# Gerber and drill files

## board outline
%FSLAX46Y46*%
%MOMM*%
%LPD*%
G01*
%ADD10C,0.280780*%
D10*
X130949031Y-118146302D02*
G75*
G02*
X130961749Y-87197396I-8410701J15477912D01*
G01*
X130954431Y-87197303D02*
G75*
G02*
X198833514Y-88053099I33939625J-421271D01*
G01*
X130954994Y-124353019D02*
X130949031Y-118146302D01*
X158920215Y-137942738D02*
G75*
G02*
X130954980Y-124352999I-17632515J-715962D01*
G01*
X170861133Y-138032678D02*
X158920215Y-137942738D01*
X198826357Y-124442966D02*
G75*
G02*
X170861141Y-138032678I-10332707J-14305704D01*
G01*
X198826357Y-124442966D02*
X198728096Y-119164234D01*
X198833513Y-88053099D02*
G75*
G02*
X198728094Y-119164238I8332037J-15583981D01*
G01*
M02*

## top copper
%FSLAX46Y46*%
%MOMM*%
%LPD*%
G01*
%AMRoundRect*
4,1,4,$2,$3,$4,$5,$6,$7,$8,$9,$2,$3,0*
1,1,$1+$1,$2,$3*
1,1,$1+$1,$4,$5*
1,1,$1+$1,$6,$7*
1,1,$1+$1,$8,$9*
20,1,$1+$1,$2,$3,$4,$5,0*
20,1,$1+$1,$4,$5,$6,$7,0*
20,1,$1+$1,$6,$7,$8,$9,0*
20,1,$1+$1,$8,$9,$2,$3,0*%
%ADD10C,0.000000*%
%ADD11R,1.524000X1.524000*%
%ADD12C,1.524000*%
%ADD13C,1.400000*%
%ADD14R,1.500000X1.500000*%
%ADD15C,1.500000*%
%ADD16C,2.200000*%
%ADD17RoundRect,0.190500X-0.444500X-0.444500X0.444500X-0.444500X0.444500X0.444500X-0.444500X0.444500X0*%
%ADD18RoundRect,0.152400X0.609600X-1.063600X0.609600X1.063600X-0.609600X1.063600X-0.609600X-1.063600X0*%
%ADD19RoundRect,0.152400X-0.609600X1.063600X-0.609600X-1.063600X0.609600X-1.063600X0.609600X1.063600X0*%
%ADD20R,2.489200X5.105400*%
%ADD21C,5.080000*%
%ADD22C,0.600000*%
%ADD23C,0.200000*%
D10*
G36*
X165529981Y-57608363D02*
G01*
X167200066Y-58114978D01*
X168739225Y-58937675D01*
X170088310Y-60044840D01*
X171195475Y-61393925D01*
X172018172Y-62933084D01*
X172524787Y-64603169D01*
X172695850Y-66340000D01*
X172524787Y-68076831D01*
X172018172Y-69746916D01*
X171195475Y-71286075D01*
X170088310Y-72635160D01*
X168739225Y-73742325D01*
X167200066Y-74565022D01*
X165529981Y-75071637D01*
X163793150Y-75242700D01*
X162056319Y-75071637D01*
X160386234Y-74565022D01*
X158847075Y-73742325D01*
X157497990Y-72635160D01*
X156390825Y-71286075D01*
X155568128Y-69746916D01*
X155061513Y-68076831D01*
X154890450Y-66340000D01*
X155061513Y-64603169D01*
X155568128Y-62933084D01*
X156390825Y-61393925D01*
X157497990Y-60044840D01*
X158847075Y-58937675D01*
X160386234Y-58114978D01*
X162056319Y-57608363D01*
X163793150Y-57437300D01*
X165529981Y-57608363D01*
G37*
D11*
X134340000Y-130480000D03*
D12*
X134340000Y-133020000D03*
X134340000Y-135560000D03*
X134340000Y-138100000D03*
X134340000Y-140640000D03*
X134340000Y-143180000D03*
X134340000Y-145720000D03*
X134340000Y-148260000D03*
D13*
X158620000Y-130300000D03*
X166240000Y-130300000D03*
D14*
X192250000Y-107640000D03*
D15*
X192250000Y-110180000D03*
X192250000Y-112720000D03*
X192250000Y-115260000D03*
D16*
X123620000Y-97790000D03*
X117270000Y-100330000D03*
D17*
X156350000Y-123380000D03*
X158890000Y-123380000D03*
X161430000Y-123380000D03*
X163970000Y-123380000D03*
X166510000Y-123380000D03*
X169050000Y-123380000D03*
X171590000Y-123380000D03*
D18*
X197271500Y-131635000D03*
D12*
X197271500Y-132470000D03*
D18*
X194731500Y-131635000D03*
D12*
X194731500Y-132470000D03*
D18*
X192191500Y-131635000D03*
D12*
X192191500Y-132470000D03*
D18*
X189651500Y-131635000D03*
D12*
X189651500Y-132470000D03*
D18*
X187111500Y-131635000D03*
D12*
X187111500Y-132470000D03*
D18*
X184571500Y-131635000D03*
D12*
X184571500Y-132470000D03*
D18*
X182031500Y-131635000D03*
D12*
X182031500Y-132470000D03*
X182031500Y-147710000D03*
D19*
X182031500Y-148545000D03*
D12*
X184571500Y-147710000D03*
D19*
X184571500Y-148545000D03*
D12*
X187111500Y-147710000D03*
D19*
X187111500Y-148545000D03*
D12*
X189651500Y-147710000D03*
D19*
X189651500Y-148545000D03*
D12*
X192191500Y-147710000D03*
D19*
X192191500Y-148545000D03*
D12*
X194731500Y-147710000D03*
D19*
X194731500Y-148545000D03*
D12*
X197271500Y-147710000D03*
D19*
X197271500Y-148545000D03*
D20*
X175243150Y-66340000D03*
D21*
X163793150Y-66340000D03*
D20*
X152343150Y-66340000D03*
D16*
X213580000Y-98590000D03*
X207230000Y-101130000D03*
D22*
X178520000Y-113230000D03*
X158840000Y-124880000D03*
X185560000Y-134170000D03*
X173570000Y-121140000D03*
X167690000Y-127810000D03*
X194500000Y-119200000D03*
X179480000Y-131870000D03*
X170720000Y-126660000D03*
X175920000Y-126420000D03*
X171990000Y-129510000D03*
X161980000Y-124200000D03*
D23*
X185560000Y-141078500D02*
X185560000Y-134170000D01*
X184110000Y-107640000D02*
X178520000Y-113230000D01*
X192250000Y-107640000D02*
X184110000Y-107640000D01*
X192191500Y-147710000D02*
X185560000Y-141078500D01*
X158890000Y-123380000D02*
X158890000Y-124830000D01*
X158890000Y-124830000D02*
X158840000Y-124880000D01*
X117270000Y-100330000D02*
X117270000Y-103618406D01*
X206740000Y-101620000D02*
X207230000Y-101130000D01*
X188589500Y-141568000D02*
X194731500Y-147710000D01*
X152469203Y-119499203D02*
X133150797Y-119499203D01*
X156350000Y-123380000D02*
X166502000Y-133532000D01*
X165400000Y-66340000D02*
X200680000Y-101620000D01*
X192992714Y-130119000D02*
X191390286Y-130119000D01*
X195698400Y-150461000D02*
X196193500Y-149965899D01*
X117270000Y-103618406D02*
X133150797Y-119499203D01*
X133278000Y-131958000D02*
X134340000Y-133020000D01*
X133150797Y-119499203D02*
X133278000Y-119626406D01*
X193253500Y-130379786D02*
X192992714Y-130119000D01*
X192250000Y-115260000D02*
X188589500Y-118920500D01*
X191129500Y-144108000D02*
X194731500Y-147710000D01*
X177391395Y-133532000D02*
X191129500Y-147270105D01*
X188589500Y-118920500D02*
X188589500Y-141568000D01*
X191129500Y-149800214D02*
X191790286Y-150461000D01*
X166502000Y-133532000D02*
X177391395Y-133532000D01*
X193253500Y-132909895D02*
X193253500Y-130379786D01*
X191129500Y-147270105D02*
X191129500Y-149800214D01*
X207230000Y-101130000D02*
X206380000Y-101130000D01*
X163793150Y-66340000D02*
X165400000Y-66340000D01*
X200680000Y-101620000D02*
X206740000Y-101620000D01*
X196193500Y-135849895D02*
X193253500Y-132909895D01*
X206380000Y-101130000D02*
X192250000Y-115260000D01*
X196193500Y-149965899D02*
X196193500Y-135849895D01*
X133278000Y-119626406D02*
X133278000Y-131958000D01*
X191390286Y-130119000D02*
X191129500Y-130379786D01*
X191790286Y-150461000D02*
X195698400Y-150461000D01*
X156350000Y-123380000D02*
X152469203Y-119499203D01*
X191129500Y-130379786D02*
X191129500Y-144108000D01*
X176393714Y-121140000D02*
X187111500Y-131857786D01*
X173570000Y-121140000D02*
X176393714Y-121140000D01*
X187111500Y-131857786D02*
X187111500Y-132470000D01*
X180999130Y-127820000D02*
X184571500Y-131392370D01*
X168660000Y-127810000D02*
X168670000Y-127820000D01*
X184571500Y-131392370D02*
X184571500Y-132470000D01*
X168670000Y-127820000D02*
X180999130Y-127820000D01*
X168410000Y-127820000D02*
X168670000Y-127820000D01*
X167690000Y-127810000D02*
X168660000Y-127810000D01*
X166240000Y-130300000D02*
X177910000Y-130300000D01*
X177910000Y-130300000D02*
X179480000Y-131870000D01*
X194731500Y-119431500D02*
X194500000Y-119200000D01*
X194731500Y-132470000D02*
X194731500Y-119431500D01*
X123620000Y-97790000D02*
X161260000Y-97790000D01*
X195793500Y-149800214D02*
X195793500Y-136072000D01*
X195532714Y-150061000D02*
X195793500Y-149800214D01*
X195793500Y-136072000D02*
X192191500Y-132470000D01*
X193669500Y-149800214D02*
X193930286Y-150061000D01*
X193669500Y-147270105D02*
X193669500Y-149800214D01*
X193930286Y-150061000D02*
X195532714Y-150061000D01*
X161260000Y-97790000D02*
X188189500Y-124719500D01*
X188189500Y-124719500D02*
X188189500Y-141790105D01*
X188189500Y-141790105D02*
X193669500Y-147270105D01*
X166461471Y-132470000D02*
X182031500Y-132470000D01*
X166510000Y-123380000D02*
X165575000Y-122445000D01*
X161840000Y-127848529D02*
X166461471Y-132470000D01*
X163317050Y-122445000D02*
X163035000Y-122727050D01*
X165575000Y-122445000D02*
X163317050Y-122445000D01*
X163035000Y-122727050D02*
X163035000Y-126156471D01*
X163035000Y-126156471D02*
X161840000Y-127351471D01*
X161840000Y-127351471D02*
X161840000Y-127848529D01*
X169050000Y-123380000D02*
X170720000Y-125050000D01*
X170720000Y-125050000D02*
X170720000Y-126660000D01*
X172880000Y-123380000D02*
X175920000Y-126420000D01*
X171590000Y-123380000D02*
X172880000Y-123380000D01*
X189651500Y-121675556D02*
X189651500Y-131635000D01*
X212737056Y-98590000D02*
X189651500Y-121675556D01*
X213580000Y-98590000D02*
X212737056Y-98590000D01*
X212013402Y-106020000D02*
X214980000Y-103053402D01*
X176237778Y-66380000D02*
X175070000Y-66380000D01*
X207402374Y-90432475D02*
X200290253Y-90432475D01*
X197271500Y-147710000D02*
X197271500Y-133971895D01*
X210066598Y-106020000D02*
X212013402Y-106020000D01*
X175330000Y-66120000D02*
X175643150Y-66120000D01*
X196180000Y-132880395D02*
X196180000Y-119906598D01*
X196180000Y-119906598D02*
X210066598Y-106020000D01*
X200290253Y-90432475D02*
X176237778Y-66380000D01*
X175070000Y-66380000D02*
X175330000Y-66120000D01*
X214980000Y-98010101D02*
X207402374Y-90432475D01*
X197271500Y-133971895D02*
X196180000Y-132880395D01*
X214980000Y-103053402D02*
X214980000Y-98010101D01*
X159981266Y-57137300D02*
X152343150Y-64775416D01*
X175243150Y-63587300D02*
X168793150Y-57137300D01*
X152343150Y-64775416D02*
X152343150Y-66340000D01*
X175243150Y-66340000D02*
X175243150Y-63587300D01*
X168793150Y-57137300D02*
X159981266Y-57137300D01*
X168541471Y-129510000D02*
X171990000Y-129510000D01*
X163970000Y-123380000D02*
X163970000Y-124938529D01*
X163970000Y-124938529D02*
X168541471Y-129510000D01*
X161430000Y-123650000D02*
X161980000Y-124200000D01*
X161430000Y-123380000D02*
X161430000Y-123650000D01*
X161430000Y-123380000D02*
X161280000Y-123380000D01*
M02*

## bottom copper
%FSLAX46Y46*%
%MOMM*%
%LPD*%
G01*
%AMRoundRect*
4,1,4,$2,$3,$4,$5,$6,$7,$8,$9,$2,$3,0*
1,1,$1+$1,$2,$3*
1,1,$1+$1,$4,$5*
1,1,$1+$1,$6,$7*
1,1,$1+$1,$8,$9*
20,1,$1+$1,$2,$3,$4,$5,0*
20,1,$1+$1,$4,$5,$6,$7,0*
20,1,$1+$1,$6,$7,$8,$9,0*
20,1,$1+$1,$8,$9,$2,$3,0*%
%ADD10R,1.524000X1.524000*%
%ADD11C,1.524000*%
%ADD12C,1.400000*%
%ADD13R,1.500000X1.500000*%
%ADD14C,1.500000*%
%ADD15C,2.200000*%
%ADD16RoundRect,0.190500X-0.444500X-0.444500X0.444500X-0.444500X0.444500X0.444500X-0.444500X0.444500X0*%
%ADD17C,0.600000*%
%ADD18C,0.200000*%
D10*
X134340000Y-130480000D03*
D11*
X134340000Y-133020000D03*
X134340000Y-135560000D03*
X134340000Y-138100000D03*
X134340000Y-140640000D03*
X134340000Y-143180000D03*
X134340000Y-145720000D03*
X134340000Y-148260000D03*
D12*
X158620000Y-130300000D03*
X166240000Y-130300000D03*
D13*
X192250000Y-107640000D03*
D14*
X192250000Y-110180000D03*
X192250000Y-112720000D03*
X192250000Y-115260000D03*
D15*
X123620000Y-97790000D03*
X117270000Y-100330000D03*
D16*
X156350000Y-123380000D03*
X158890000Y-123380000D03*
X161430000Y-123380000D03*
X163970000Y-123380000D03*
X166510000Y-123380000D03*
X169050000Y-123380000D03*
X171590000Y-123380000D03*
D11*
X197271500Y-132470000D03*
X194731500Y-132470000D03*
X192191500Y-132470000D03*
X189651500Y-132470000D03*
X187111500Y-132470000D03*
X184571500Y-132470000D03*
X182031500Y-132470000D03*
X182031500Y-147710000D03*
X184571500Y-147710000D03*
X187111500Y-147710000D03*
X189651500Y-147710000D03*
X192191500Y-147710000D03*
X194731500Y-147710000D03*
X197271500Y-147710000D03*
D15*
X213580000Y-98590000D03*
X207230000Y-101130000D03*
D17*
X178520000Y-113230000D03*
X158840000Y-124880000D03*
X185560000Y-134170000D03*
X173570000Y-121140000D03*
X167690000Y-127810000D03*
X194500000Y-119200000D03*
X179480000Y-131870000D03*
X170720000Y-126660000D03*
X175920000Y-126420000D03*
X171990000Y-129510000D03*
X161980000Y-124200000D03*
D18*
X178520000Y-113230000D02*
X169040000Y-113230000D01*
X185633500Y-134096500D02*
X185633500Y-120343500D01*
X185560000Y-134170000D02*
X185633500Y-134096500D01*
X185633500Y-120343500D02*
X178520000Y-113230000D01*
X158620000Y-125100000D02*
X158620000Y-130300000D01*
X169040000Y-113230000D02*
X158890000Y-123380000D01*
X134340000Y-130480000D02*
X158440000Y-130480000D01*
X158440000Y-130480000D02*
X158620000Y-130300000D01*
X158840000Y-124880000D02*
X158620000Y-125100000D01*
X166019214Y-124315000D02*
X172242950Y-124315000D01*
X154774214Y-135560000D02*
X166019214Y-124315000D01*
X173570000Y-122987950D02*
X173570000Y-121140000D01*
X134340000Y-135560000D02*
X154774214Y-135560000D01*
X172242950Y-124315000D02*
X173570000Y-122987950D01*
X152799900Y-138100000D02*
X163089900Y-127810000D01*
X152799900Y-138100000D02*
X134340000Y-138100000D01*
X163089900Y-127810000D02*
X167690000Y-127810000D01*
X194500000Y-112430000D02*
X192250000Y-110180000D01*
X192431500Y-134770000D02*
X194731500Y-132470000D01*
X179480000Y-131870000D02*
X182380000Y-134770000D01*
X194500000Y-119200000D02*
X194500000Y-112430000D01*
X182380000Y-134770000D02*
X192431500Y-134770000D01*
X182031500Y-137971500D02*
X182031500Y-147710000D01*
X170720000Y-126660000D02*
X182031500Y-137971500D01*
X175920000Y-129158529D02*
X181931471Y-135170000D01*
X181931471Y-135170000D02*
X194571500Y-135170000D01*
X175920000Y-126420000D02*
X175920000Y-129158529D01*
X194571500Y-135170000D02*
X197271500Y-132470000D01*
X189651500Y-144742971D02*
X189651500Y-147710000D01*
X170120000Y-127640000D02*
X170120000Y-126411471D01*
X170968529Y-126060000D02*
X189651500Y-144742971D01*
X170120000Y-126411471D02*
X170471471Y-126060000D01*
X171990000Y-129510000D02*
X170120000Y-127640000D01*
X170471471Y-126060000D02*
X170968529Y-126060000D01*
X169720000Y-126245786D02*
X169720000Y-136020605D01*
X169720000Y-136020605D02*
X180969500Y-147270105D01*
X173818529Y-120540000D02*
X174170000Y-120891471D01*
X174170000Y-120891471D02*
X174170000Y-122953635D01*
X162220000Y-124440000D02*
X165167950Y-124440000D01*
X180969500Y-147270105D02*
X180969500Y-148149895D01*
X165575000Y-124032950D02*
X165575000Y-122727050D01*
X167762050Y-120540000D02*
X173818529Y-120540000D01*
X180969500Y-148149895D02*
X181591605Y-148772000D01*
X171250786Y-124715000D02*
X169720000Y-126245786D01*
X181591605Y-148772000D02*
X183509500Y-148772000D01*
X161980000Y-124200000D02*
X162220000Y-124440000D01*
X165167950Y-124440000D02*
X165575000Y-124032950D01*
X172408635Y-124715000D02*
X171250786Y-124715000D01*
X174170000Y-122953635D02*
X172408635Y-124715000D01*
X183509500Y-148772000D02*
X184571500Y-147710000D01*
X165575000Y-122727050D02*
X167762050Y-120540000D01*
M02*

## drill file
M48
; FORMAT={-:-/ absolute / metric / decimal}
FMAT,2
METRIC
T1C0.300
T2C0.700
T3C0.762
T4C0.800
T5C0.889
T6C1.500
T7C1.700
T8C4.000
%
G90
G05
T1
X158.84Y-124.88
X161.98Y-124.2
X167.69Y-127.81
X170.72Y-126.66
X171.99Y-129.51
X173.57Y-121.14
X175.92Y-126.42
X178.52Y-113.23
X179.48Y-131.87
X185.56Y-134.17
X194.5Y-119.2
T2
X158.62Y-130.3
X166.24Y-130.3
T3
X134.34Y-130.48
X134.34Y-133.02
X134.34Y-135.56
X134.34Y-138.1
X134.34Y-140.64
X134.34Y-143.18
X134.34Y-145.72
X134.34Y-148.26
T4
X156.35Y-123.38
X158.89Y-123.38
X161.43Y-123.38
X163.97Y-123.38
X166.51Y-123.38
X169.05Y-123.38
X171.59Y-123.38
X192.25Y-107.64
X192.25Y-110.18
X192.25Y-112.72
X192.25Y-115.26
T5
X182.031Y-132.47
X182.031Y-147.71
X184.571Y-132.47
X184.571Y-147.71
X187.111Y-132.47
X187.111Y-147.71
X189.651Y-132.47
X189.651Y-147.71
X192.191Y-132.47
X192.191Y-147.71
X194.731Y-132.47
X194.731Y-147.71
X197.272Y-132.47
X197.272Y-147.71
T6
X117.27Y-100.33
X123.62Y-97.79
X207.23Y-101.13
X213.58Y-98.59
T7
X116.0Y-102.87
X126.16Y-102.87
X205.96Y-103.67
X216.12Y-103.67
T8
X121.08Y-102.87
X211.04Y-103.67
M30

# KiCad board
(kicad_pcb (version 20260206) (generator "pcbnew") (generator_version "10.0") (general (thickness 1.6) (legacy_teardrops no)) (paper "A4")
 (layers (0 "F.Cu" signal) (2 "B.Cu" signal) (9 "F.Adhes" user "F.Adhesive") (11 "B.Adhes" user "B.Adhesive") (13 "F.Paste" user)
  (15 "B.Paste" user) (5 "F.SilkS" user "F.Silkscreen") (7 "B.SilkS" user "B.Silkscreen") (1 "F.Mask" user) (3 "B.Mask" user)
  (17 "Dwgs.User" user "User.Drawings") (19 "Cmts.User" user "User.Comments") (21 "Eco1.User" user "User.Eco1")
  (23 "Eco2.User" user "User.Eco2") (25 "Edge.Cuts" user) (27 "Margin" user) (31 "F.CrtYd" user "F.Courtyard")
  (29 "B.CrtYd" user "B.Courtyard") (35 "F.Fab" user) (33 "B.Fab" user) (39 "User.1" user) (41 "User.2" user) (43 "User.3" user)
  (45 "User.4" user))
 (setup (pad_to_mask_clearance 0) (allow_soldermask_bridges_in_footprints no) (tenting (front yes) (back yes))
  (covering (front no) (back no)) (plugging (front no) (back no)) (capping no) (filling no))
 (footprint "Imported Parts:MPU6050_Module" (layer "F.Cu") (at 134.34 130.48)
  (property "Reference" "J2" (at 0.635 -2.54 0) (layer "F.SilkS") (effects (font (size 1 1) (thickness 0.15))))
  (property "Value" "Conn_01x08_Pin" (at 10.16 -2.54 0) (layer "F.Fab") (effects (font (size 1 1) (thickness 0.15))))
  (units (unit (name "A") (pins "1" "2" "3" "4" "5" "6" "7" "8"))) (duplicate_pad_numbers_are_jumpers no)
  (pad "1" thru_hole rect (at 0 0) (size 1.524 1.524) (drill 0.762) (layers "*.Cu" "*.Mask") (remove_unused_layers no) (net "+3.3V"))
  (pad "2" thru_hole circle (at 0 2.54) (size 1.524 1.524) (drill 0.762) (layers "*.Cu" "*.Mask") (remove_unused_layers no) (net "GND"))
  (pad "3" thru_hole circle (at 0 5.08) (size 1.524 1.524) (drill 0.762) (layers "*.Cu" "*.Mask") (remove_unused_layers no) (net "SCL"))
  (pad "4" thru_hole circle (at 0 7.62) (size 1.524 1.524) (drill 0.762) (layers "*.Cu" "*.Mask") (remove_unused_layers no) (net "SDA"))
  (pad "5" thru_hole circle (at 0 10.16) (size 1.524 1.524) (drill 0.762) (layers "*.Cu" "*.Mask") (remove_unused_layers no)
   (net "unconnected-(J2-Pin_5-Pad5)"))
  (pad "6" thru_hole circle (at 0 12.7) (size 1.524 1.524) (drill 0.762) (layers "*.Cu" "*.Mask") (remove_unused_layers no)
   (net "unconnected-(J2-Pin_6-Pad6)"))
  (pad "7" thru_hole circle (at 0 15.24) (size 1.524 1.524) (drill 0.762) (layers "*.Cu" "*.Mask") (remove_unused_layers no)
   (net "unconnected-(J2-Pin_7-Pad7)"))
  (pad "8" thru_hole circle (at 0 17.78) (size 1.524 1.524) (drill 0.762) (layers "*.Cu" "*.Mask") (remove_unused_layers no)
   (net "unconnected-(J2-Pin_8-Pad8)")))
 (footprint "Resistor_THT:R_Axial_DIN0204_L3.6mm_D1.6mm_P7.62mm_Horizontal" (layer "F.Cu") (at 158.62 130.3)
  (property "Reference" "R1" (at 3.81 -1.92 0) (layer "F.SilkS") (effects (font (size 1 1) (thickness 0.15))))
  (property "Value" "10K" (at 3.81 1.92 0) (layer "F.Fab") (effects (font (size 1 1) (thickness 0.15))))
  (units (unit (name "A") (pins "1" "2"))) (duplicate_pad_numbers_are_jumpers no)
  (pad "1" thru_hole circle (at 0 0) (size 1.4 1.4) (drill 0.7) (layers "*.Cu" "*.Mask") (remove_unused_layers no) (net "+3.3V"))
  (pad "2" thru_hole circle (at 7.62 0) (size 1.4 1.4) (drill 0.7) (layers "*.Cu" "*.Mask") (remove_unused_layers no) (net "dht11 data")))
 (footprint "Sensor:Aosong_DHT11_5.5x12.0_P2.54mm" (layer "F.Cu") (at 192.25 107.64)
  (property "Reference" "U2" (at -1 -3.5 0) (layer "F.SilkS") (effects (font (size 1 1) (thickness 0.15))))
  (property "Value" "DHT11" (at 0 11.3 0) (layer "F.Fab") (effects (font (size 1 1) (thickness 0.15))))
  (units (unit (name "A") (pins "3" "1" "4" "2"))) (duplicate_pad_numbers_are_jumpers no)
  (pad "1" thru_hole rect (at 0 0) (size 1.5 1.5) (drill 0.8) (layers "*.Cu" "*.Mask") (remove_unused_layers no) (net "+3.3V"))
  (pad "2" thru_hole circle (at 0 2.54) (size 1.5 1.5) (drill 0.8) (layers "*.Cu" "*.Mask") (remove_unused_layers no) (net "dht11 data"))
  (pad "3" thru_hole circle (at 0 5.08) (size 1.5 1.5) (drill 0.8) (layers "*.Cu" "*.Mask") (remove_unused_layers no)
   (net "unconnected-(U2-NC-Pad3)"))
  (pad "4" thru_hole circle (at 0 7.62) (size 1.5 1.5) (drill 0.8) (layers "*.Cu" "*.Mask") (remove_unused_layers no) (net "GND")))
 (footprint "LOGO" (layer "F.Cu") (at 148.84 83.94)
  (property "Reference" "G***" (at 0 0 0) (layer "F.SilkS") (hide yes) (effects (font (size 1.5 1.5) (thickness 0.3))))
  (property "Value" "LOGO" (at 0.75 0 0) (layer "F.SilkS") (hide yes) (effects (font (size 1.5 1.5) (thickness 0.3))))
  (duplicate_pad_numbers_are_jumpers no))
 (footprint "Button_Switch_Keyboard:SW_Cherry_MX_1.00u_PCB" (layer "F.Cu") (at 123.62 97.79)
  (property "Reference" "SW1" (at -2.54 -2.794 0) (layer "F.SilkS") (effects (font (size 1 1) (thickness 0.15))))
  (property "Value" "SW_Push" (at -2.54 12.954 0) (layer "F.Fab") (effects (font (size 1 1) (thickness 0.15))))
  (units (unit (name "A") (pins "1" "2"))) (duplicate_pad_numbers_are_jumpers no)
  (pad "" np_thru_hole circle (at -7.62 5.08) (size 1.7 1.7) (drill 1.7) (layers "*.Cu" "*.Mask"))
  (pad "" np_thru_hole circle (at -2.54 5.08) (size 4 4) (drill 4) (layers "*.Cu" "*.Mask"))
  (pad "" np_thru_hole circle (at 2.54 5.08) (size 1.7 1.7) (drill 1.7) (layers "*.Cu" "*.Mask"))
  (pad "1" thru_hole circle (at 0 0) (size 2.2 2.2) (drill 1.5) (layers "*.Cu" "*.Mask") (remove_unused_layers no) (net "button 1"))
  (pad "2" thru_hole circle (at -6.35 2.54) (size 2.2 2.2) (drill 1.5) (layers "*.Cu" "*.Mask") (remove_unused_layers no) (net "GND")))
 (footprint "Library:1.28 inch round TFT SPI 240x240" (layer "F.Cu") (at 163.97 98.94)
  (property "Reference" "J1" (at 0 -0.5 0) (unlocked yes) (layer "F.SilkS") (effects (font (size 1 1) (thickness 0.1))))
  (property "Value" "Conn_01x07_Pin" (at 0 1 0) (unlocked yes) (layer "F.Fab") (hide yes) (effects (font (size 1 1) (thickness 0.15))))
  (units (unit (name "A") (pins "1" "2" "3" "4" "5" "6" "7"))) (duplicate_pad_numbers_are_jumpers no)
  (pad "1" thru_hole roundrect (at -7.62 24.44) (size 1.27 1.27) (drill 0.8) (layers "*.Cu" "*.Mask") (remove_unused_layers no)
   (roundrect_rratio 0.15) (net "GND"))
  (pad "2" thru_hole roundrect (at -5.08 24.44) (size 1.27 1.27) (drill 0.8) (layers "*.Cu" "*.Mask") (remove_unused_layers no)
   (roundrect_rratio 0.15) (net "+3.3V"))
  (pad "3" thru_hole roundrect (at -2.54 24.44) (size 1.27 1.27) (drill 0.8) (layers "*.Cu" "*.Mask") (remove_unused_layers no)
   (roundrect_rratio 0.15) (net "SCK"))
  (pad "4" thru_hole roundrect (at 0 24.44) (size 1.27 1.27) (drill 0.8) (layers "*.Cu" "*.Mask") (remove_unused_layers no)
   (roundrect_rratio 0.15) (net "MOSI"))
  (pad "5" thru_hole roundrect (at 2.54 24.44) (size 1.27 1.27) (drill 0.8) (layers "*.Cu" "*.Mask") (remove_unused_layers no)
   (roundrect_rratio 0.15) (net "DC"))
  (pad "6" thru_hole roundrect (at 5.08 24.44) (size 1.27 1.27) (drill 0.8) (layers "*.Cu" "*.Mask") (remove_unused_layers no)
   (roundrect_rratio 0.15) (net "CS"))
  (pad "7" thru_hole roundrect (at 7.62 24.44) (size 1.27 1.27) (drill 0.8) (layers "*.Cu" "*.Mask") (remove_unused_layers no)
   (roundrect_rratio 0.15) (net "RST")))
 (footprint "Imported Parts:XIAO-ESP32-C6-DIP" (layer "F.Cu") (at 189.6515 140.09)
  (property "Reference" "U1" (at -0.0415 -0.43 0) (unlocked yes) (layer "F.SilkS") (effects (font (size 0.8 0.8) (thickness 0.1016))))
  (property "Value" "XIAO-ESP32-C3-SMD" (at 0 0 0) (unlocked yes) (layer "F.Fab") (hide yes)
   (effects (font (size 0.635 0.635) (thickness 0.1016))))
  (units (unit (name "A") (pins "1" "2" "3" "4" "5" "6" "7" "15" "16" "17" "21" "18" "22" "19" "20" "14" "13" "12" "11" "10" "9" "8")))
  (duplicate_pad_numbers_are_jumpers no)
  (pad "1" smd roundrect (at 7.62 -8.455 90) (size 2.432 1.524) (layers "F.Cu" "F.Mask") (roundrect_rratio 0.1) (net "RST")
   (thermal_bridge_angle 45))
  (pad "1" thru_hole circle (at 7.62 -7.62 90) (size 1.524 1.524) (drill 0.889) (layers "*.Cu" "*.Mask") (remove_unused_layers no)
   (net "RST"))
  (pad "2" smd roundrect (at 5.08 -8.455 90) (size 2.432 1.524) (layers "F.Cu" "F.Mask") (roundrect_rratio 0.1) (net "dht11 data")
   (thermal_bridge_angle 45))
  (pad "2" thru_hole circle (at 5.08 -7.62 90) (size 1.524 1.524) (drill 0.889) (layers "*.Cu" "*.Mask") (remove_unused_layers no)
   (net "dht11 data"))
  (pad "3" smd roundrect (at 2.54 -8.455 90) (size 2.432 1.524) (layers "F.Cu" "F.Mask") (roundrect_rratio 0.1) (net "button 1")
   (thermal_bridge_angle 45))
  (pad "3" thru_hole circle (at 2.54 -7.62 90) (size 1.524 1.524) (drill 0.889) (layers "*.Cu" "*.Mask") (remove_unused_layers no)
   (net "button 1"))
  (pad "4" smd roundrect (at 0 -8.455 90) (size 2.432 1.524) (layers "F.Cu" "F.Mask") (roundrect_rratio 0.1) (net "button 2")
   (thermal_bridge_angle 45))
  (pad "4" thru_hole circle (at 0 -7.62 90) (size 1.524 1.524) (drill 0.889) (layers "*.Cu" "*.Mask") (remove_unused_layers no)
   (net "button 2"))
  (pad "5" smd roundrect (at -2.54 -8.455 90) (size 2.432 1.524) (layers "F.Cu" "F.Mask") (roundrect_rratio 0.1) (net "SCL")
   (thermal_bridge_angle 45))
  (pad "5" thru_hole circle (at -2.54 -7.62 90) (size 1.524 1.524) (drill 0.889) (layers "*.Cu" "*.Mask") (remove_unused_layers no)
   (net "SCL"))
  (pad "6" smd roundrect (at -5.08 -8.455 90) (size 2.432 1.524) (layers "F.Cu" "F.Mask") (roundrect_rratio 0.1) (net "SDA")
   (thermal_bridge_angle 45))
  (pad "6" thru_hole circle (at -5.08 -7.62 90) (size 1.524 1.524) (drill 0.889) (layers "*.Cu" "*.Mask") (remove_unused_layers no)
   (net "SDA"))
  (pad "7" smd roundrect (at -7.62 -8.455 90) (size 2.432 1.524) (layers "F.Cu" "F.Mask") (roundrect_rratio 0.1) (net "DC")
   (thermal_bridge_angle 45))
  (pad "7" thru_hole circle (at -7.62 -7.62 90) (size 1.524 1.524) (drill 0.889) (layers "*.Cu" "*.Mask") (remove_unused_layers no)
   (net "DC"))
  (pad "8" thru_hole circle (at -7.62 7.62 270) (size 1.524 1.524) (drill 0.889) (layers "*.Cu" "*.Mask") (remove_unused_layers no)
   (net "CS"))
  (pad "8" smd roundrect (at -7.62 8.455 270) (size 2.432 1.524) (layers "F.Cu" "F.Mask") (roundrect_rratio 0.1) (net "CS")
   (thermal_bridge_angle 45))
  (pad "9" thru_hole circle (at -5.08 7.62 270) (size 1.524 1.524) (drill 0.889) (layers "*.Cu" "*.Mask") (remove_unused_layers no)
   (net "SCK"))
  (pad "9" smd roundrect (at -5.08 8.455 270) (size 2.432 1.524) (layers "F.Cu" "F.Mask") (roundrect_rratio 0.1) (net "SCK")
   (thermal_bridge_angle 45))
  (pad "10" thru_hole circle (at -2.54 7.62 270) (size 1.524 1.524) (drill 0.889) (layers "*.Cu" "*.Mask") (remove_unused_layers no)
   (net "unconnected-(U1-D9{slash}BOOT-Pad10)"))
  (pad "10" smd roundrect (at -2.54 8.455 270) (size 2.432 1.524) (layers "F.Cu" "F.Mask") (roundrect_rratio 0.1)
   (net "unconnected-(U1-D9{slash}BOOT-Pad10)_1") (thermal_bridge_angle 45))
  (pad "11" thru_hole circle (at 0 7.62 270) (size 1.524 1.524) (drill 0.889) (layers "*.Cu" "*.Mask") (remove_unused_layers no)
   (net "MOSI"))
  (pad "11" smd roundrect (at 0 8.455 270) (size 2.432 1.524) (layers "F.Cu" "F.Mask") (roundrect_rratio 0.1) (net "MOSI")
   (thermal_bridge_angle 45))
  (pad "12" thru_hole circle (at 2.54 7.62 270) (size 1.524 1.524) (drill 0.889) (layers "*.Cu" "*.Mask") (remove_unused_layers no)
   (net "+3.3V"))
  (pad "12" smd roundrect (at 2.54 8.455 270) (size 2.432 1.524) (layers "F.Cu" "F.Mask") (roundrect_rratio 0.1) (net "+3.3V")
   (thermal_bridge_angle 45))
  (pad "13" thru_hole circle (at 5.08 7.62 270) (size 1.524 1.524) (drill 0.889) (layers "*.Cu" "*.Mask") (remove_unused_layers no)
   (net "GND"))
  (pad "13" smd roundrect (at 5.08 8.455 270) (size 2.432 1.524) (layers "F.Cu" "F.Mask") (roundrect_rratio 0.1) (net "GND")
   (thermal_bridge_angle 45))
  (pad "14" thru_hole circle (at 7.62 7.62 270) (size 1.524 1.524) (drill 0.889) (layers "*.Cu" "*.Mask") (remove_unused_layers no)
   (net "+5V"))
  (pad "14" smd roundrect (at 7.62 8.455 270) (size 2.432 1.524) (layers "F.Cu" "F.Mask") (roundrect_rratio 0.1) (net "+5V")
   (thermal_bridge_angle 45)))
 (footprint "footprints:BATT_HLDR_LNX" (layer "F.Cu") (at 163.79315 66.34 180)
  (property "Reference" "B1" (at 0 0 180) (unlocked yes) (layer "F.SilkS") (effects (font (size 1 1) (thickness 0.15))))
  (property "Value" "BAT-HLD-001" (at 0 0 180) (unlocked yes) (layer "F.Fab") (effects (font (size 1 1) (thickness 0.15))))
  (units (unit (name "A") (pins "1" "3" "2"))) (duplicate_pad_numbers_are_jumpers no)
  (fp_poly
   (pts (xy 8.9027 0) (xy 8.731637 -1.736831) (xy 8.225022 -3.406916) (xy 7.402325 -4.946075) (xy 6.29516 -6.29516) (xy 4.946075 -7.402325)
    (xy 3.406916 -8.225022) (xy 1.736831 -8.731637) (xy 0 -8.9027) (xy -1.736831 -8.731637) (xy -3.406916 -8.225022)
    (xy -4.946075 -7.402325) (xy -6.29516 -6.29516) (xy -7.402325 -4.946075) (xy -8.225022 -3.406916) (xy -8.731637 -1.736831)
    (xy -8.9027 0) (xy -8.731637 1.736831) (xy -8.225022 3.406916) (xy -7.402325 4.946075) (xy -6.29516 6.29516) (xy -4.946075 7.402325)
    (xy -3.406916 8.225022) (xy -1.736831 8.731637) (xy 0 8.9027) (xy 1.736831 8.731637) (xy 3.406916 8.225022) (xy 4.946075 7.402325)
    (xy 6.29516 6.29516) (xy 7.402325 4.946075) (xy 8.225022 3.406916) (xy 8.731637 1.736831))
   (stroke (width 0) (type solid)) (fill yes) (layer "F.Cu"))
  (pad "1" smd rect (at -11.45 0 180) (size 2.4892 5.1054) (layers "F.Cu" "F.Mask" "F.Paste") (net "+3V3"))
  (pad "2" smd circle (at 0 0 180) (size 5.08 5.08) (layers "F.Cu" "F.Mask" "F.Paste") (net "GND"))
  (pad "3" smd rect (at 11.45 0 180) (size 2.4892 5.1054) (layers "F.Cu" "F.Mask" "F.Paste") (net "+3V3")))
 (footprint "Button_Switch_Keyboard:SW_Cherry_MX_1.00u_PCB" (layer "F.Cu") (at 213.58 98.59)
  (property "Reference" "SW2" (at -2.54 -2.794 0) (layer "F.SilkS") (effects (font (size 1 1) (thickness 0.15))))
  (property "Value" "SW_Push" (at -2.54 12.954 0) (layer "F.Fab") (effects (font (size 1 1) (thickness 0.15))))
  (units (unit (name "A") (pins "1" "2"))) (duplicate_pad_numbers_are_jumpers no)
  (pad "" np_thru_hole circle (at -7.62 5.08) (size 1.7 1.7) (drill 1.7) (layers "*.Cu" "*.Mask"))
  (pad "" np_thru_hole circle (at -2.54 5.08) (size 4 4) (drill 4) (layers "*.Cu" "*.Mask"))
  (pad "" np_thru_hole circle (at 2.54 5.08) (size 1.7 1.7) (drill 1.7) (layers "*.Cu" "*.Mask"))
  (pad "1" thru_hole circle (at 0 0) (size 2.2 2.2) (drill 1.5) (layers "*.Cu" "*.Mask") (remove_unused_layers no) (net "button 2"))
  (pad "2" thru_hole circle (at -6.35 2.54) (size 2.2 2.2) (drill 1.5) (layers "*.Cu" "*.Mask") (remove_unused_layers no) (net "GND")))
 (gr_arc (start 130.949031 118.146302) (mid 104.922837 102.661154) (end 130.961752 87.197391) (stroke (width 0.28078) (type solid))
  (layer "Edge.Cuts"))
 (gr_arc (start 130.954431 87.197303) (mid 165.321951 53.679032) (end 198.833513 88.053099) (stroke (width 0.28078) (type solid))
  (layer "Edge.Cuts"))
 (gr_line (start 130.954994 124.353019) (end 130.949031 118.146302) (stroke (width 0.28078) (type solid)) (layer "Edge.Cuts"))
 (gr_arc (start 158.920215 137.942738) (mid 133.574606 154.530907) (end 130.954994 124.353019) (stroke (width 0.28078) (type solid))
  (layer "Edge.Cuts"))
 (gr_line (start 170.861133 138.032678) (end 158.920215 137.942738) (stroke (width 0.28078) (type solid)) (layer "Edge.Cuts"))
 (gr_arc (start 198.826357 124.442966) (mid 196.20674 154.620857) (end 170.861133 138.032678) (stroke (width 0.28078) (type solid))
  (layer "Edge.Cuts"))
 (gr_line (start 198.826357 124.442966) (end 198.728096 119.164234) (stroke (width 0.28078) (type solid)) (layer "Edge.Cuts"))
 (gr_arc (start 198.833513 88.053099) (mid 224.83698 103.696965) (end 198.728096 119.164234) (stroke (width 0.28078) (type solid))
  (layer "Edge.Cuts"))
 (segment (start 185.56 141.0785) (end 185.56 134.17) (width 0.2) (layer "F.Cu") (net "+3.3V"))
 (segment (start 184.11 107.64) (end 178.52 113.23) (width 0.2) (layer "F.Cu") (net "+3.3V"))
 (segment (start 192.25 107.64) (end 184.11 107.64) (width 0.2) (layer "F.Cu") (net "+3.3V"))
 (segment (start 192.1915 147.71) (end 185.56 141.0785) (width 0.2) (layer "F.Cu") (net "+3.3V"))
 (segment (start 158.89 123.38) (end 158.89 124.83) (width 0.2) (layer "F.Cu") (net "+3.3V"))
 (segment (start 158.89 124.83) (end 158.84 124.88) (width 0.2) (layer "F.Cu") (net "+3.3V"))
 (via (at 178.52 113.23) (size 0.6) (drill 0.3) (layers "F.Cu" "B.Cu") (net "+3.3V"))
 (via (at 158.84 124.88) (size 0.6) (drill 0.3) (layers "F.Cu" "B.Cu") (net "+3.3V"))
 (via (at 185.56 134.17) (size 0.6) (drill 0.3) (layers "F.Cu" "B.Cu") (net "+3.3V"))
 (segment (start 178.52 113.23) (end 169.04 113.23) (width 0.2) (layer "B.Cu") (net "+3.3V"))
 (segment (start 185.6335 134.0965) (end 185.6335 120.3435) (width 0.2) (layer "B.Cu") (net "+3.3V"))
 (segment (start 185.56 134.17) (end 185.6335 134.0965) (width 0.2) (layer "B.Cu") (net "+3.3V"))
 (segment (start 185.6335 120.3435) (end 178.52 113.23) (width 0.2) (layer "B.Cu") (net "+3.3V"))
 (segment (start 158.62 125.1) (end 158.62 130.3) (width 0.2) (layer "B.Cu") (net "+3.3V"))
 (segment (start 169.04 113.23) (end 158.89 123.38) (width 0.2) (layer "B.Cu") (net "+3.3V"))
 (segment (start 134.34 130.48) (end 158.44 130.48) (width 0.2) (layer "B.Cu") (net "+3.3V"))
 (segment (start 158.44 130.48) (end 158.62 130.3) (width 0.2) (layer "B.Cu") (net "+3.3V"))
 (segment (start 158.84 124.88) (end 158.62 125.1) (width 0.2) (layer "B.Cu") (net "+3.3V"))
 (segment (start 117.27 100.33) (end 117.27 103.618406) (width 0.2) (layer "F.Cu") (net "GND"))
 (segment (start 206.74 101.62) (end 207.23 101.13) (width 0.2) (layer "F.Cu") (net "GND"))
 (segment (start 188.5895 141.568) (end 194.7315 147.71) (width 0.2) (layer "F.Cu") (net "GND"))
 (segment (start 152.469203 119.499203) (end 133.150797 119.499203) (width 0.2) (layer "F.Cu") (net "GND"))
 (segment (start 156.35 123.38) (end 166.502 133.532) (width 0.2) (layer "F.Cu") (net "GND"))
 (segment (start 165.4 66.34) (end 200.68 101.62) (width 0.2) (layer "F.Cu") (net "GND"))
 (segment (start 192.992714 130.119) (end 191.390286 130.119) (width 0.2) (layer "F.Cu") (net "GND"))
 (segment (start 195.6984 150.461) (end 196.1935 149.965899) (width 0.2) (layer "F.Cu") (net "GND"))
 (segment (start 117.27 103.618406) (end 133.150797 119.499203) (width 0.2) (layer "F.Cu") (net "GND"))
 (segment (start 133.278 131.958) (end 134.34 133.02) (width 0.2) (layer "F.Cu") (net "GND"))
 (segment (start 133.150797 119.499203) (end 133.278 119.626406) (width 0.2) (layer "F.Cu") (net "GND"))
 (segment (start 193.2535 130.379786) (end 192.992714 130.119) (width 0.2) (layer "F.Cu") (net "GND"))
 (segment (start 192.25 115.26) (end 188.5895 118.9205) (width 0.2) (layer "F.Cu") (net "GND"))
 (segment (start 191.1295 144.108) (end 194.7315 147.71) (width 0.2) (layer "F.Cu") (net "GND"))
 (segment (start 177.391395 133.532) (end 191.1295 147.270105) (width 0.2) (layer "F.Cu") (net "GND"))
 (segment (start 188.5895 118.9205) (end 188.5895 141.568) (width 0.2) (layer "F.Cu") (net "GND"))
 (segment (start 191.1295 149.800214) (end 191.790286 150.461) (width 0.2) (layer "F.Cu") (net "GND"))
 (segment (start 166.502 133.532) (end 177.391395 133.532) (width 0.2) (layer "F.Cu") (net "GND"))
 (segment (start 193.2535 132.909895) (end 193.2535 130.379786) (width 0.2) (layer "F.Cu") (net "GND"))
 (segment (start 191.1295 147.270105) (end 191.1295 149.800214) (width 0.2) (layer "F.Cu") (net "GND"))
 (segment (start 207.23 101.13) (end 206.38 101.13) (width 0.2) (layer "F.Cu") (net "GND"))
 (segment (start 163.79315 66.34) (end 165.4 66.34) (width 0.2) (layer "F.Cu") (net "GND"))
 (segment (start 200.68 101.62) (end 206.74 101.62) (width 0.2) (layer "F.Cu") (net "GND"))
 (segment (start 196.1935 135.849895) (end 193.2535 132.909895) (width 0.2) (layer "F.Cu") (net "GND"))
 (segment (start 206.38 101.13) (end 192.25 115.26) (width 0.2) (layer "F.Cu") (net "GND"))
 (segment (start 196.1935 149.965899) (end 196.1935 135.849895) (width 0.2) (layer "F.Cu") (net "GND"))
 (segment (start 133.278 119.626406) (end 133.278 131.958) (width 0.2) (layer "F.Cu") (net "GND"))
 (segment (start 191.390286 130.119) (end 191.1295 130.379786) (width 0.2) (layer "F.Cu") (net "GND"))
 (segment (start 191.790286 150.461) (end 195.6984 150.461) (width 0.2) (layer "F.Cu") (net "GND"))
 (segment (start 156.35 123.38) (end 152.469203 119.499203) (width 0.2) (layer "F.Cu") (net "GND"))
 (segment (start 191.1295 130.379786) (end 191.1295 144.108) (width 0.2) (layer "F.Cu") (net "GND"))
 (segment (start 176.393714 121.14) (end 187.1115 131.857786) (width 0.2) (layer "F.Cu") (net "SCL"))
 (segment (start 173.57 121.14) (end 176.393714 121.14) (width 0.2) (layer "F.Cu") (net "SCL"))
 (segment (start 187.1115 131.857786) (end 187.1115 132.47) (width 0.2) (layer "F.Cu") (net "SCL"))
 (via (at 173.57 121.14) (size 0.6) (drill 0.3) (layers "F.Cu" "B.Cu") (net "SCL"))
 (segment (start 166.019214 124.315) (end 172.24295 124.315) (width 0.2) (layer "B.Cu") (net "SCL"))
 (segment (start 154.774214 135.56) (end 166.019214 124.315) (width 0.2) (layer "B.Cu") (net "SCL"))
 (segment (start 173.57 122.98795) (end 173.57 121.14) (width 0.2) (layer "B.Cu") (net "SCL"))
 (segment (start 134.34 135.56) (end 154.774214 135.56) (width 0.2) (layer "B.Cu") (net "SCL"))
 (segment (start 172.24295 124.315) (end 173.57 122.98795) (width 0.2) (layer "B.Cu") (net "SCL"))
 (segment (start 180.99913 127.82) (end 184.5715 131.39237) (width 0.2) (layer "F.Cu") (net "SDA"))
 (segment (start 168.66 127.81) (end 168.67 127.82) (width 0.2) (layer "F.Cu") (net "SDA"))
 (segment (start 184.5715 131.39237) (end 184.5715 132.47) (width 0.2) (layer "F.Cu") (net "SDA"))
 (segment (start 168.67 127.82) (end 180.99913 127.82) (width 0.2) (layer "F.Cu") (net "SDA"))
 (segment (start 168.41 127.82) (end 168.67 127.82) (width 0.2) (layer "F.Cu") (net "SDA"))
 (segment (start 167.69 127.81) (end 168.66 127.81) (width 0.2) (layer "F.Cu") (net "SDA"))
 (via (at 167.69 127.81) (size 0.6) (drill 0.3) (layers "F.Cu" "B.Cu") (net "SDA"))
 (segment (start 152.7999 138.1) (end 163.0899 127.81) (width 0.2) (layer "B.Cu") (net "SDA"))
 (segment (start 152.7999 138.1) (end 134.34 138.1) (width 0.2) (layer "B.Cu") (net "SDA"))
 (segment (start 163.0899 127.81) (end 167.69 127.81) (width 0.2) (layer "B.Cu") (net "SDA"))
 (segment (start 166.24 130.3) (end 177.91 130.3) (width 0.2) (layer "F.Cu") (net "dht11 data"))
 (segment (start 177.91 130.3) (end 179.48 131.87) (width 0.2) (layer "F.Cu") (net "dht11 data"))
 (segment (start 194.7315 119.4315) (end 194.5 119.2) (width 0.2) (layer "F.Cu") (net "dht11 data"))
 (segment (start 194.7315 132.47) (end 194.7315 119.4315) (width 0.2) (layer "F.Cu") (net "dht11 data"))
 (via (at 194.5 119.2) (size 0.6) (drill 0.3) (layers "F.Cu" "B.Cu") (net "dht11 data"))
 (via (at 179.48 131.87) (size 0.6) (drill 0.3) (layers "F.Cu" "B.Cu") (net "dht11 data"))
 (segment (start 194.5 112.43) (end 192.25 110.18) (width 0.2) (layer "B.Cu") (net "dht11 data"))
 (segment (start 192.4315 134.77) (end 194.7315 132.47) (width 0.2) (layer "B.Cu") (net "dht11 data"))
 (segment (start 179.48 131.87) (end 182.38 134.77) (width 0.2) (layer "B.Cu") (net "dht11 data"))
 (segment (start 194.5 119.2) (end 194.5 112.43) (width 0.2) (layer "B.Cu") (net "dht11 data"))
 (segment (start 182.38 134.77) (end 192.4315 134.77) (width 0.2) (layer "B.Cu") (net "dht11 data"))
 (segment (start 123.62 97.79) (end 161.26 97.79) (width 0.2) (layer "F.Cu") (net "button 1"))
 (segment (start 195.7935 149.800214) (end 195.7935 136.072) (width 0.2) (layer "F.Cu") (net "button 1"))
 (segment (start 195.532714 150.061) (end 195.7935 149.800214) (width 0.2) (layer "F.Cu") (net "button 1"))
 (segment (start 195.7935 136.072) (end 192.1915 132.47) (width 0.2) (layer "F.Cu") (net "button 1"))
 (segment (start 193.6695 149.800214) (end 193.930286 150.061) (width 0.2) (layer "F.Cu") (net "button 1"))
 (segment (start 193.6695 147.270105) (end 193.6695 149.800214) (width 0.2) (layer "F.Cu") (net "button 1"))
 (segment (start 193.930286 150.061) (end 195.532714 150.061) (width 0.2) (layer "F.Cu") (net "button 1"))
 (segment (start 161.26 97.79) (end 188.1895 124.7195) (width 0.2) (layer "F.Cu") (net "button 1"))
 (segment (start 188.1895 124.7195) (end 188.1895 141.790105) (width 0.2) (layer "F.Cu") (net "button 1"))
 (segment (start 188.1895 141.790105) (end 193.6695 147.270105) (width 0.2) (layer "F.Cu") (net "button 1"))
 (segment (start 166.461471 132.47) (end 182.0315 132.47) (width 0.2) (layer "F.Cu") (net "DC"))
 (segment (start 166.51 123.38) (end 165.575 122.445) (width 0.2) (layer "F.Cu") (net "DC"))
 (segment (start 161.84 127.848529) (end 166.461471 132.47) (width 0.2) (layer "F.Cu") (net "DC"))
 (segment (start 163.31705 122.445) (end 163.035 122.72705) (width 0.2) (layer "F.Cu") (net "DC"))
 (segment (start 165.575 122.445) (end 163.31705 122.445) (width 0.2) (layer "F.Cu") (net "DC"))
 (segment (start 163.035 122.72705) (end 163.035 126.156471) (width 0.2) (layer "F.Cu") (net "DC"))
 (segment (start 163.035 126.156471) (end 161.84 127.351471) (width 0.2) (layer "F.Cu") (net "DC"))
 (segment (start 161.84 127.351471) (end 161.84 127.848529) (width 0.2) (layer "F.Cu") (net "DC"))
 (segment (start 169.05 123.38) (end 170.72 125.05) (width 0.2) (layer "F.Cu") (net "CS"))
 (segment (start 170.72 125.05) (end 170.72 126.66) (width 0.2) (layer "F.Cu") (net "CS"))
 (via (at 170.72 126.66) (size 0.6) (drill 0.3) (layers "F.Cu" "B.Cu") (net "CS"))
 (segment (start 182.0315 137.9715) (end 182.0315 147.71) (width 0.2) (layer "B.Cu") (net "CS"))
 (segment (start 170.72 126.66) (end 182.0315 137.9715) (width 0.2) (layer "B.Cu") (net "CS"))
 (segment (start 172.88 123.38) (end 175.92 126.42) (width 0.2) (layer "F.Cu") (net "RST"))
 (segment (start 171.59 123.38) (end 172.88 123.38) (width 0.2) (layer "F.Cu") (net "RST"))
 (via (at 175.92 126.42) (size 0.6) (drill 0.3) (layers "F.Cu" "B.Cu") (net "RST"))
 (segment (start 175.92 129.158529) (end 181.931471 135.17) (width 0.2) (layer "B.Cu") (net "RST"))
 (segment (start 181.931471 135.17) (end 194.5715 135.17) (width 0.2) (layer "B.Cu") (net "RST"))
 (segment (start 175.92 126.42) (end 175.92 129.158529) (width 0.2) (layer "B.Cu") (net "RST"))
 (segment (start 194.5715 135.17) (end 197.2715 132.47) (width 0.2) (layer "B.Cu") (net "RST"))
 (segment (start 189.6515 121.675556) (end 189.6515 131.635) (width 0.2) (layer "F.Cu") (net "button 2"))
 (segment (start 212.737056 98.59) (end 189.6515 121.675556) (width 0.2) (layer "F.Cu") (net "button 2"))
 (segment (start 213.58 98.59) (end 212.737056 98.59) (width 0.2) (layer "F.Cu") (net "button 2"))
 (segment (start 212.013402 106.02) (end 214.98 103.053402) (width 0.2) (layer "F.Cu") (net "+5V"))
 (segment (start 176.237778 66.38) (end 175.07 66.38) (width 0.2) (layer "F.Cu") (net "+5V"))
 (segment (start 207.402374 90.432475) (end 200.290253 90.432475) (width 0.2) (layer "F.Cu") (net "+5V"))
 (segment (start 197.2715 147.71) (end 197.2715 133.971895) (width 0.2) (layer "F.Cu") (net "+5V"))
 (segment (start 210.066598 106.02) (end 212.013402 106.02) (width 0.2) (layer "F.Cu") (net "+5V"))
 (segment (start 175.33 66.12) (end 175.64315 66.12) (width 0.2) (layer "F.Cu") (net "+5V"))
 (segment (start 196.18 132.880395) (end 196.18 119.906598) (width 0.2) (layer "F.Cu") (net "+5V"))
 (segment (start 196.18 119.906598) (end 210.066598 106.02) (width 0.2) (layer "F.Cu") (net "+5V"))
 (segment (start 200.290253 90.432475) (end 176.237778 66.38) (width 0.2) (layer "F.Cu") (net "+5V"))
 (segment (start 175.07 66.38) (end 175.33 66.12) (width 0.2) (layer "F.Cu") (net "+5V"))
 (segment (start 214.98 98.010101) (end 207.402374 90.432475) (width 0.2) (layer "F.Cu") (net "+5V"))
 (segment (start 197.2715 133.971895) (end 196.18 132.880395) (width 0.2) (layer "F.Cu") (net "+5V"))
 (segment (start 214.98 103.053402) (end 214.98 98.010101) (width 0.2) (layer "F.Cu") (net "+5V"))
 (segment (start 159.981266 57.1373) (end 152.34315 64.775416) (width 0.2) (layer "F.Cu") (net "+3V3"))
 (segment (start 175.24315 63.5873) (end 168.79315 57.1373) (width 0.2) (layer "F.Cu") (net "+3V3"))
 (segment (start 152.34315 64.775416) (end 152.34315 66.34) (width 0.2) (layer "F.Cu") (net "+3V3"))
 (segment (start 175.24315 66.34) (end 175.24315 63.5873) (width 0.2) (layer "F.Cu") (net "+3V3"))
 (segment (start 168.79315 57.1373) (end 159.981266 57.1373) (width 0.2) (layer "F.Cu") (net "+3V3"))
 (segment (start 168.541471 129.51) (end 171.99 129.51) (width 0.2) (layer "F.Cu") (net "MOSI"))
 (segment (start 163.97 123.38) (end 163.97 124.938529) (width 0.2) (layer "F.Cu") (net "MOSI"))
 (segment (start 163.97 124.938529) (end 168.541471 129.51) (width 0.2) (layer "F.Cu") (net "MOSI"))
 (via (at 171.99 129.51) (size 0.6) (drill 0.3) (layers "F.Cu" "B.Cu") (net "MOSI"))
 (segment (start 189.6515 144.742971) (end 189.6515 147.71) (width 0.2) (layer "B.Cu") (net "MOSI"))
 (segment (start 170.12 127.64) (end 170.12 126.411471) (width 0.2) (layer "B.Cu") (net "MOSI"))
 (segment (start 170.968529 126.06) (end 189.6515 144.742971) (width 0.2) (layer "B.Cu") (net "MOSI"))
 (segment (start 170.12 126.411471) (end 170.471471 126.06) (width 0.2) (layer "B.Cu") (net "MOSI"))
 (segment (start 171.99 129.51) (end 170.12 127.64) (width 0.2) (layer "B.Cu") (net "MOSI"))
 (segment (start 170.471471 126.06) (end 170.968529 126.06) (width 0.2) (layer "B.Cu") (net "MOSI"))
 (segment (start 161.43 123.65) (end 161.98 124.2) (width 0.2) (layer "F.Cu") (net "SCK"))
 (segment (start 161.43 123.38) (end 161.43 123.65) (width 0.2) (layer "F.Cu") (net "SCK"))
 (segment (start 161.43 123.38) (end 161.28 123.38) (width 0.2) (layer "F.Cu") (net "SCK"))
 (via (at 161.98 124.2) (size 0.6) (drill 0.3) (layers "F.Cu" "B.Cu") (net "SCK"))
 (segment (start 169.72 126.245786) (end 169.72 136.020605) (width 0.2) (layer "B.Cu") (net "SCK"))
 (segment (start 169.72 136.020605) (end 180.9695 147.270105) (width 0.2) (layer "B.Cu") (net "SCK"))
 (segment (start 173.818529 120.54) (end 174.17 120.891471) (width 0.2) (layer "B.Cu") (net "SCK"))
 (segment (start 174.17 120.891471) (end 174.17 122.953635) (width 0.2) (layer "B.Cu") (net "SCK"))
 (segment (start 162.22 124.44) (end 165.16795 124.44) (width 0.2) (layer "B.Cu") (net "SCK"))
 (segment (start 180.9695 147.270105) (end 180.9695 148.149895) (width 0.2) (layer "B.Cu") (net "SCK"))
 (segment (start 165.575 124.03295) (end 165.575 122.72705) (width 0.2) (layer "B.Cu") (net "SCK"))
 (segment (start 167.76205 120.54) (end 173.818529 120.54) (width 0.2) (layer "B.Cu") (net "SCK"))
 (segment (start 180.9695 148.149895) (end 181.591605 148.772) (width 0.2) (layer "B.Cu") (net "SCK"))
 (segment (start 171.250786 124.715) (end 169.72 126.245786) (width 0.2) (layer "B.Cu") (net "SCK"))
 (segment (start 181.591605 148.772) (end 183.5095 148.772) (width 0.2) (layer "B.Cu") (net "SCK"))
 (segment (start 161.98 124.2) (end 162.22 124.44) (width 0.2) (layer "B.Cu") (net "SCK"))
 (segment (start 165.16795 124.44) (end 165.575 124.03295) (width 0.2) (layer "B.Cu") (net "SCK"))
 (segment (start 172.408635 124.715) (end 171.250786 124.715) (width 0.2) (layer "B.Cu") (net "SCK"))
 (segment (start 174.17 122.953635) (end 172.408635 124.715) (width 0.2) (layer "B.Cu") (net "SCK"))
 (segment (start 183.5095 148.772) (end 184.5715 147.71) (width 0.2) (layer "B.Cu") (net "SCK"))
 (segment (start 165.575 122.72705) (end 167.76205 120.54) (width 0.2) (layer "B.Cu") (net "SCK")))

